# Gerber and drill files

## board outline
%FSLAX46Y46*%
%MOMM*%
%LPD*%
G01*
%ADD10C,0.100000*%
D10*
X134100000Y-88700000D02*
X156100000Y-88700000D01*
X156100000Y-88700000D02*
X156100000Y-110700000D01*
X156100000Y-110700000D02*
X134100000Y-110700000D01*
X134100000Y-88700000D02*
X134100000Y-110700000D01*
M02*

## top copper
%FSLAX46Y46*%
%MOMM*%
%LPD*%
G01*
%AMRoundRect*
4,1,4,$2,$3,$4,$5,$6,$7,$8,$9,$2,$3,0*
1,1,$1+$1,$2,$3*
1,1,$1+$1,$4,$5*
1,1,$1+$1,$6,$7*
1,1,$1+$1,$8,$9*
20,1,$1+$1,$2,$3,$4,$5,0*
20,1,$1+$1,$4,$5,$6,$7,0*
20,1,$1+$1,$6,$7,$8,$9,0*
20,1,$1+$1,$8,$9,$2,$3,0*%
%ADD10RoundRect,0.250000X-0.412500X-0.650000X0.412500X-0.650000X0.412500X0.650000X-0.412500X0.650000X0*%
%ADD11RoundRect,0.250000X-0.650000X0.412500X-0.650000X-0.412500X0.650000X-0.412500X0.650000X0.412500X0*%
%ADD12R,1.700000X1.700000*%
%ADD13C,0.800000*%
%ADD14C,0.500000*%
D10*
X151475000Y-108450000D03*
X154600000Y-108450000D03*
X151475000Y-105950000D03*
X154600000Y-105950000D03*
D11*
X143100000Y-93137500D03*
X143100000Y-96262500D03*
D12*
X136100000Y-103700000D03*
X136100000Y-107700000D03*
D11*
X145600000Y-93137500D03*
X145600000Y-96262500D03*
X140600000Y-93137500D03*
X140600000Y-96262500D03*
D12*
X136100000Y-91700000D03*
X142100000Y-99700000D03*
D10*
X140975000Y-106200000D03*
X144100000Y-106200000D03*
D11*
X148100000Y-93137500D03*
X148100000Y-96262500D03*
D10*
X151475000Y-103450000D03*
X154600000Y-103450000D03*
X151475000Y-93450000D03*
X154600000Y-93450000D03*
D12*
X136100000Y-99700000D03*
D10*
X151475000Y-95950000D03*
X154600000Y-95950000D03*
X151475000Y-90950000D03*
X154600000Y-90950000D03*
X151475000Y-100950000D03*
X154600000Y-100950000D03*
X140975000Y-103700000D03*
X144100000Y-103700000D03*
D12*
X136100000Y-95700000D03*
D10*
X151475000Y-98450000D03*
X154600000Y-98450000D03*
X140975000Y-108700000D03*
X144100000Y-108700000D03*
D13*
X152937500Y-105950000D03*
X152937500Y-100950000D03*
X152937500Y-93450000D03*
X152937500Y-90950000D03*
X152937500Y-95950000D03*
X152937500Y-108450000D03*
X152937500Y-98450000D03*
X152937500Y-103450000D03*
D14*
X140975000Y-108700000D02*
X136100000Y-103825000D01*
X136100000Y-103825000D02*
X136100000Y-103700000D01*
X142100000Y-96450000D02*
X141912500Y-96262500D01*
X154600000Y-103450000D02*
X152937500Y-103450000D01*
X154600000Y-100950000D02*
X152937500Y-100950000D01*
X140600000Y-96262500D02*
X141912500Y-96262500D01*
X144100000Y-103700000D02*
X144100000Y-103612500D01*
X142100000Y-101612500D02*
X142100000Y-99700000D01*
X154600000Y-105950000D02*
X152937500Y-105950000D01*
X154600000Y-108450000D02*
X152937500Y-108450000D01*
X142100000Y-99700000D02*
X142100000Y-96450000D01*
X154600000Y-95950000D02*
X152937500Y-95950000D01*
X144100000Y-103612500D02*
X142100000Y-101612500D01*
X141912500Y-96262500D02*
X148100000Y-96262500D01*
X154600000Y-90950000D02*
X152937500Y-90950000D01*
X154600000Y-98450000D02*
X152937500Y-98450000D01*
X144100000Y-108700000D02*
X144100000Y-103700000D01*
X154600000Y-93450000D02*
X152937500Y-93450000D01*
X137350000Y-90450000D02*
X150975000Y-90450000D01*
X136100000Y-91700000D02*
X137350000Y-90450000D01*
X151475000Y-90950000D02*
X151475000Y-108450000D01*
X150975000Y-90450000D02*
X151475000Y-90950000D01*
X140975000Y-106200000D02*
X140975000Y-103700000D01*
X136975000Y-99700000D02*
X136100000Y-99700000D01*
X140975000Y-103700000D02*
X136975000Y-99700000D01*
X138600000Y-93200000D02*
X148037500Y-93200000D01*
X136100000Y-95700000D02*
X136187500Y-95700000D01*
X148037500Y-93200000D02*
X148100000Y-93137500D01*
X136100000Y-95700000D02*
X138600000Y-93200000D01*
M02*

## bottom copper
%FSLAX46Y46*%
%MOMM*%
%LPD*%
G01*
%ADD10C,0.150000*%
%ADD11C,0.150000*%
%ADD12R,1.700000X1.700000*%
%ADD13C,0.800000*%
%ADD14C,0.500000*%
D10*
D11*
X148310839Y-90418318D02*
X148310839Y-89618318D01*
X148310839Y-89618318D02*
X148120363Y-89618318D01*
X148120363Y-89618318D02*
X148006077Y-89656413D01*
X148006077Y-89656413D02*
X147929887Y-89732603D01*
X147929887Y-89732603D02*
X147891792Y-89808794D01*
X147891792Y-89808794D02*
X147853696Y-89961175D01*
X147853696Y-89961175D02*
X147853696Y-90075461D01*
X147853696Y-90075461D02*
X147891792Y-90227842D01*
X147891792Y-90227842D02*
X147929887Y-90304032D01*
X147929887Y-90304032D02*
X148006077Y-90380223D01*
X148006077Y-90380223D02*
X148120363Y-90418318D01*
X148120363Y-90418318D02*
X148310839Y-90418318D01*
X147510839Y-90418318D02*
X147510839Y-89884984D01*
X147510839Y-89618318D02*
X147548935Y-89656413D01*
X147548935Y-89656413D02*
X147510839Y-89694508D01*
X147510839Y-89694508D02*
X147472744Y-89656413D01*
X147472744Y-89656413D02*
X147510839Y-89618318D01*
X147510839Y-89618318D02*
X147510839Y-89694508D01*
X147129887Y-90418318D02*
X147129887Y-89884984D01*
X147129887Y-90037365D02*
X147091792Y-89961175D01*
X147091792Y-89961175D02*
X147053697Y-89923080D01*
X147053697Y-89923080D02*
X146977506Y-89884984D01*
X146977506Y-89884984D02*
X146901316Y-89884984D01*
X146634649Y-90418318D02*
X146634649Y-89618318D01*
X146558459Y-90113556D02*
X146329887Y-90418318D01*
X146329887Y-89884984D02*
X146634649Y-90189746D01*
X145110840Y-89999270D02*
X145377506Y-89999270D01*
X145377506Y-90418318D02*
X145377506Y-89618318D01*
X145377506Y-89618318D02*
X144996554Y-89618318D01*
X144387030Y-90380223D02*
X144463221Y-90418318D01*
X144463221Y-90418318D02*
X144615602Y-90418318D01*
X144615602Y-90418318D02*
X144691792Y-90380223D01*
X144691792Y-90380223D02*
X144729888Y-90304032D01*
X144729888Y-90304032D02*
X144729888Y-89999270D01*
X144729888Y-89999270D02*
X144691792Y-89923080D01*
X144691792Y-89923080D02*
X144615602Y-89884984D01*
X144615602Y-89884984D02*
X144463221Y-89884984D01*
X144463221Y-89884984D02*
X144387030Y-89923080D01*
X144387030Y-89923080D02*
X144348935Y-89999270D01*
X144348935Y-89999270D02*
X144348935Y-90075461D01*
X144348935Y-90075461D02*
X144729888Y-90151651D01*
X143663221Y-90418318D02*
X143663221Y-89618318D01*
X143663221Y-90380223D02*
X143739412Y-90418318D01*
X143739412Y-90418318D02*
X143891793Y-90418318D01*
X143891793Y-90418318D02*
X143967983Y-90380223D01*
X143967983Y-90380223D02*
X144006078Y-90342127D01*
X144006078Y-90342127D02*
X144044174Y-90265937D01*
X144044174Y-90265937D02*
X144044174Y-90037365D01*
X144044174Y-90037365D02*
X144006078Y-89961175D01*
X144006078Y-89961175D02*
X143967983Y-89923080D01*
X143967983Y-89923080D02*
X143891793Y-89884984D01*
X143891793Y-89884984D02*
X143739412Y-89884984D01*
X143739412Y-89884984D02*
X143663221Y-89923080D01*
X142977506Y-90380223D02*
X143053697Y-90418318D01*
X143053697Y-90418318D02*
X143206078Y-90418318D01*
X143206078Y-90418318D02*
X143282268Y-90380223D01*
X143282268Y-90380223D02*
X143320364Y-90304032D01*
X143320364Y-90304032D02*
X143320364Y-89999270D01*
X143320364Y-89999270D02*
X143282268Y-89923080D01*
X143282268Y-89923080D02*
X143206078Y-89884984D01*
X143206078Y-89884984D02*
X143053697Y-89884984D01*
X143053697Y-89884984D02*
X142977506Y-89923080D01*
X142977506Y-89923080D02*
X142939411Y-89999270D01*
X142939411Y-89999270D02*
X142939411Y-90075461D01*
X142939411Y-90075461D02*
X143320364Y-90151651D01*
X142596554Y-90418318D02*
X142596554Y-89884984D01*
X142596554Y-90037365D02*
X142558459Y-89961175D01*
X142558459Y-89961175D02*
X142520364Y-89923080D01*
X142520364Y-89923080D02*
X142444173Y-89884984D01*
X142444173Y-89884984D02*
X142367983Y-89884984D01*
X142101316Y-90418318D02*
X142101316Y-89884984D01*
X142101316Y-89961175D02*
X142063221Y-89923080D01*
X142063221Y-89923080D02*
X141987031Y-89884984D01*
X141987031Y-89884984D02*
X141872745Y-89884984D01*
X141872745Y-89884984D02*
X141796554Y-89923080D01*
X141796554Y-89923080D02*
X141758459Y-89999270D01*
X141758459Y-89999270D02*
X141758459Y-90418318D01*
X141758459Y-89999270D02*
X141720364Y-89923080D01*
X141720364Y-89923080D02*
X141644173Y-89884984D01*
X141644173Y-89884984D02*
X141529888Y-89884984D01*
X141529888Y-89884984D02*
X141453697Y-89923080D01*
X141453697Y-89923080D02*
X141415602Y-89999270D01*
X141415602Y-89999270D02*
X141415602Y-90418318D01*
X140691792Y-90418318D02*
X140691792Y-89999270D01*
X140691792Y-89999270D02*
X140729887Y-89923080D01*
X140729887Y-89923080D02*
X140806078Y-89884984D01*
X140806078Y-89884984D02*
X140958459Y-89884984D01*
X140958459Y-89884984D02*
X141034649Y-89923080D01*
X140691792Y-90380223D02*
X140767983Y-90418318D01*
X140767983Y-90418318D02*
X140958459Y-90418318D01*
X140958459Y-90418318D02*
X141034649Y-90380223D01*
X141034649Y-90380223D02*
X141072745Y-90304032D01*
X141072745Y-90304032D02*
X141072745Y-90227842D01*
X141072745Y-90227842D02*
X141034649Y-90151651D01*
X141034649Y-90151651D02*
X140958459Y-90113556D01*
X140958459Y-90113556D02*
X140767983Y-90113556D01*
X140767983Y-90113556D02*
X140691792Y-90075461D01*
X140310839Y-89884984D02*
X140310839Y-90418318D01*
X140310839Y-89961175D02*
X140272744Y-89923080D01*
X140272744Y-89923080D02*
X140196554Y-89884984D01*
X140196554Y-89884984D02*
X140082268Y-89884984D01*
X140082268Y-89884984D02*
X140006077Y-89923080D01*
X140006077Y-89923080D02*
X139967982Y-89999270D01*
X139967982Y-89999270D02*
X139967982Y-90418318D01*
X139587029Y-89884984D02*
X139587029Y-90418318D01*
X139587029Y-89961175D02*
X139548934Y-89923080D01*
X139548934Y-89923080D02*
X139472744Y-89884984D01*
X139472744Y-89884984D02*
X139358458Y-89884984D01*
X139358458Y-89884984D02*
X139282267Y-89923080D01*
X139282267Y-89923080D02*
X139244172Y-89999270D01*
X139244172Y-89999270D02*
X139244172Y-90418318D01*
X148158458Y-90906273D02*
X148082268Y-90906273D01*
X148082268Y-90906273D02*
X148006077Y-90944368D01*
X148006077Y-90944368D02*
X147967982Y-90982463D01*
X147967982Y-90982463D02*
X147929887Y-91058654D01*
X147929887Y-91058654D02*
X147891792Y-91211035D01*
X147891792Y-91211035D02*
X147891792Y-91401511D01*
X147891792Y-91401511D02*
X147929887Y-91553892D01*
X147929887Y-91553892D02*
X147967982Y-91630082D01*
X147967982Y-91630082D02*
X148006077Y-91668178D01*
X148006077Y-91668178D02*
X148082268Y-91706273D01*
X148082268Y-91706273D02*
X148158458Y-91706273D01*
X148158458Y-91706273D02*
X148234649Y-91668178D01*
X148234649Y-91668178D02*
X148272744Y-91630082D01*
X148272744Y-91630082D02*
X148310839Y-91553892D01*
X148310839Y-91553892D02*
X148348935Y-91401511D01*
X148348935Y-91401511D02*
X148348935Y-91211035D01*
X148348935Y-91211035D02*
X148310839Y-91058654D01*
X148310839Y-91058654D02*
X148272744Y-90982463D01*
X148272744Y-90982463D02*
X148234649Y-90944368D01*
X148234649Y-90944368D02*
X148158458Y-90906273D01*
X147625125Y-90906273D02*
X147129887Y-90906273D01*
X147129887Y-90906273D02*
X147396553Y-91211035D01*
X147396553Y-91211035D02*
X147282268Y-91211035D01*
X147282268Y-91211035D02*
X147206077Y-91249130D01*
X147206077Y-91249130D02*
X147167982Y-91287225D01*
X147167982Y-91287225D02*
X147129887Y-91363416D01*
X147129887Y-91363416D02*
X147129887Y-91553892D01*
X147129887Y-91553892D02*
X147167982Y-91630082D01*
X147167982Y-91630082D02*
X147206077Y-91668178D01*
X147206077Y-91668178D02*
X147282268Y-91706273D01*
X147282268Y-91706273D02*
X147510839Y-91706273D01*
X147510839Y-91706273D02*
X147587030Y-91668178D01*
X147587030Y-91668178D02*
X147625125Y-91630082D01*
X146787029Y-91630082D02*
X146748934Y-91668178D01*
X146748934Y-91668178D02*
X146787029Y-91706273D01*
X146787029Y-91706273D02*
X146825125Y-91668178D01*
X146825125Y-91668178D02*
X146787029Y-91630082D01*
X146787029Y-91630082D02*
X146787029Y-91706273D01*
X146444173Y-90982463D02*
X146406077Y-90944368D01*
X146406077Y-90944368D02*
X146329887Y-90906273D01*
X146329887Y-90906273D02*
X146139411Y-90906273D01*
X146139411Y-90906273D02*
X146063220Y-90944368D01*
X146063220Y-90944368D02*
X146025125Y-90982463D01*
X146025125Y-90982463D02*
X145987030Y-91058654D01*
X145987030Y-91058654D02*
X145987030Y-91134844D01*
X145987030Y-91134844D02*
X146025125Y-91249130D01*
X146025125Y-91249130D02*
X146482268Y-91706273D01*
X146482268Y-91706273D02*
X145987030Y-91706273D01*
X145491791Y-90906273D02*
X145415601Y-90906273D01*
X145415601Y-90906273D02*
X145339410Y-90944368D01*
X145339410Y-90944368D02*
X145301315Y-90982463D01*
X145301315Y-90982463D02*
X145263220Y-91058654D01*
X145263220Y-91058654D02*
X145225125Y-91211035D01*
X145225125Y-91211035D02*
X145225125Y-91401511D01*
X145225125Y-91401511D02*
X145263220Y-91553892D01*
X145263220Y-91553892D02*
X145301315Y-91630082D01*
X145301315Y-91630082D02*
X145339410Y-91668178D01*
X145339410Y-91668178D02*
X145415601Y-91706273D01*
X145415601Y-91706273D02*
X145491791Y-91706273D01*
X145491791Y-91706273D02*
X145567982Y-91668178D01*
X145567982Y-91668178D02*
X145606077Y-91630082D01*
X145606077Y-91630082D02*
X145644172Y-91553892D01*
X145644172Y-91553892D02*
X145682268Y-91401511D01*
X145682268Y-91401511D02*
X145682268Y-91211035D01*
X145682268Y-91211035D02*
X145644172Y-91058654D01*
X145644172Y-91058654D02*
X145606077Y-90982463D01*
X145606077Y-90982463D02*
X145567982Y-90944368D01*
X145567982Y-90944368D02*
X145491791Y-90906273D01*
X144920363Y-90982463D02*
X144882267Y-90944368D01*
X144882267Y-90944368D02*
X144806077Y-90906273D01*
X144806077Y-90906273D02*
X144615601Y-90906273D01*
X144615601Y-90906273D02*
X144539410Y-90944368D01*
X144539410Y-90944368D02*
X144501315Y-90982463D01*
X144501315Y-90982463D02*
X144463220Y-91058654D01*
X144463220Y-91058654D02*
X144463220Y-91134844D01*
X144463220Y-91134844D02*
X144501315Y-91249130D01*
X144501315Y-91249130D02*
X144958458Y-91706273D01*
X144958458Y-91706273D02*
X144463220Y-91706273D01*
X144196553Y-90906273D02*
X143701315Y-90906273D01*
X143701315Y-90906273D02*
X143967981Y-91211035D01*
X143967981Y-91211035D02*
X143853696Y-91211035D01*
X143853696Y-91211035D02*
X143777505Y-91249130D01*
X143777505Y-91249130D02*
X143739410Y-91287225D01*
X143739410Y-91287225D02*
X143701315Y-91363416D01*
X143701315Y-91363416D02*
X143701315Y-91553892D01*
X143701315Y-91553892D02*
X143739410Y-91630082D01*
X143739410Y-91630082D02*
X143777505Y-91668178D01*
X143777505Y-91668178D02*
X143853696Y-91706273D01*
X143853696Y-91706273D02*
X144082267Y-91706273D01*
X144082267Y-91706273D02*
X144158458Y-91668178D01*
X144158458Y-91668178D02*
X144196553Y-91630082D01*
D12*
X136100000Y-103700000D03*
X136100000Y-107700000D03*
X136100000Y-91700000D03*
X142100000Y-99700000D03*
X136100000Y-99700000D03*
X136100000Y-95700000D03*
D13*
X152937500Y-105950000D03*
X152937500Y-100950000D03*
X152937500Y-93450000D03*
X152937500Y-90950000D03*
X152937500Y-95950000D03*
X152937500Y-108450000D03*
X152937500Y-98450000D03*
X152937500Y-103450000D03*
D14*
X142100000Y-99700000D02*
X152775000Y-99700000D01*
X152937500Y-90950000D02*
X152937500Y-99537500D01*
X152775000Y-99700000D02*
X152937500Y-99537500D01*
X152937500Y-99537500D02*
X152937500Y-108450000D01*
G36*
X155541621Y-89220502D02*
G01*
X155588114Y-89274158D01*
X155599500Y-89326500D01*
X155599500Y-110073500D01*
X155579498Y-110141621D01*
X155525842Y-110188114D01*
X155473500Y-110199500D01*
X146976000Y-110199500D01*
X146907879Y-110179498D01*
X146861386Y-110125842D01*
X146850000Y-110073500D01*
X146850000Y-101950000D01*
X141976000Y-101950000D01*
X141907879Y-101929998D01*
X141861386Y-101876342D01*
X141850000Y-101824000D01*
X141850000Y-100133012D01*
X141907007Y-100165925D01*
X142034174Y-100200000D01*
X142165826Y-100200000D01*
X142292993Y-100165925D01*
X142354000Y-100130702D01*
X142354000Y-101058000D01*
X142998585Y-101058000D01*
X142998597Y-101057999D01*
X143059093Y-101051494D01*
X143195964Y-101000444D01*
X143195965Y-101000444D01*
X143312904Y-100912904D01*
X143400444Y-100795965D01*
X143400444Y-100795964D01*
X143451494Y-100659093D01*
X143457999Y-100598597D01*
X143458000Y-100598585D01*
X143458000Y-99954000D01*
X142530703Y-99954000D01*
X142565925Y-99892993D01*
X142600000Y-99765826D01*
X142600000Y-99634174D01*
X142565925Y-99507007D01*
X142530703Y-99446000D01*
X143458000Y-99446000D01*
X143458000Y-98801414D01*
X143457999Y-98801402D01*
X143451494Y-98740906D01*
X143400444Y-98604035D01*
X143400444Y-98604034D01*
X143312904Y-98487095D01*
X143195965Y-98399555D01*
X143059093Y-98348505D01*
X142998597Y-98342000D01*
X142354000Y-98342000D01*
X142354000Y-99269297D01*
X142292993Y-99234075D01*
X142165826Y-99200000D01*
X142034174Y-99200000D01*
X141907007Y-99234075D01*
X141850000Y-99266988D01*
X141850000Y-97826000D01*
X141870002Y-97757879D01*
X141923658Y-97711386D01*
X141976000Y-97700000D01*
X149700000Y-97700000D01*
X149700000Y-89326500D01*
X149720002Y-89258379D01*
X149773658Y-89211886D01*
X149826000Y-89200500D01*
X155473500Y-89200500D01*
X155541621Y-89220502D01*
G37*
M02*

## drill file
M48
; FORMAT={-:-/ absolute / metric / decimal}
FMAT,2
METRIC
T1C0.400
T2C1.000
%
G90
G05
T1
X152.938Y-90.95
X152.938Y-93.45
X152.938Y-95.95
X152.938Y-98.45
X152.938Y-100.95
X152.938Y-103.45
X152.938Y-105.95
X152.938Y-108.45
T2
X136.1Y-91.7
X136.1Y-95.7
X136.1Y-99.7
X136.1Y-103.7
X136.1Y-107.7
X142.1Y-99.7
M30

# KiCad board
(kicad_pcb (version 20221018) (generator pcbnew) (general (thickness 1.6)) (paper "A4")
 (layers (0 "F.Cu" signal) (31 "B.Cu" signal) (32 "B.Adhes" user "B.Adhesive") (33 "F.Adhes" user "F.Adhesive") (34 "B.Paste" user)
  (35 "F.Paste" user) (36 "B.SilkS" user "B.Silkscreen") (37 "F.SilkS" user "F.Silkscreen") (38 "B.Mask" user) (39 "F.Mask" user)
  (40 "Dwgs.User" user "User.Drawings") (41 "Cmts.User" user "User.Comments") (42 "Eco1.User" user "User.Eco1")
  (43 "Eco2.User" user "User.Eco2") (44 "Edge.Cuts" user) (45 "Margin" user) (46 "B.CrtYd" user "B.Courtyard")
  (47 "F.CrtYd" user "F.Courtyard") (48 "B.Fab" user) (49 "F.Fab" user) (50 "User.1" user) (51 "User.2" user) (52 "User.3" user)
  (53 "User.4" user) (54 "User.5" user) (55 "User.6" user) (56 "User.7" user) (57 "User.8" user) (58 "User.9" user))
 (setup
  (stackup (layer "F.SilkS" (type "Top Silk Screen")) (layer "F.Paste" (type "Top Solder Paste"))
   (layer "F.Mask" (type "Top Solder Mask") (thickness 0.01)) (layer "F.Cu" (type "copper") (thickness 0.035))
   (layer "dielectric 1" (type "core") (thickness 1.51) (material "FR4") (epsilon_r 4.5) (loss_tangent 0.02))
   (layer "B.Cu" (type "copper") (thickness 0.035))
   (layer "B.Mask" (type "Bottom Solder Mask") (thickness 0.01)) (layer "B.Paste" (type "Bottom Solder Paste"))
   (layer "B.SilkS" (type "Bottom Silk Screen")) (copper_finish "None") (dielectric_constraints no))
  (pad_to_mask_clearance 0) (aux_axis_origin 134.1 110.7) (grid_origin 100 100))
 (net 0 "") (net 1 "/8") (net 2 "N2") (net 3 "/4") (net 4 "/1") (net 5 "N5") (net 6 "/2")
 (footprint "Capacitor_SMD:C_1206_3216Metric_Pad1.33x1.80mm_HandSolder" (layer "F.Cu") (at 153.0375 108.45)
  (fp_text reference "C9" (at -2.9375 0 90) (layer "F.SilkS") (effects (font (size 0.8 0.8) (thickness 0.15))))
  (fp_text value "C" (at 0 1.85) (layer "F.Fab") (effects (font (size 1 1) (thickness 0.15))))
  (pad "1" smd roundrect (at -1.5625 0) (size 1.325 1.8) (layers "F.Cu" "F.Paste" "F.Mask") (roundrect_rratio 0.1886792453) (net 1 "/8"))
  (pad "2" smd roundrect (at 1.5625 0) (size 1.325 1.8) (layers "F.Cu" "F.Paste" "F.Mask") (roundrect_rratio 0.1886792453) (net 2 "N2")))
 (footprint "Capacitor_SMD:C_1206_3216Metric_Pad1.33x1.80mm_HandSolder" (layer "F.Cu") (at 153.0375 105.95)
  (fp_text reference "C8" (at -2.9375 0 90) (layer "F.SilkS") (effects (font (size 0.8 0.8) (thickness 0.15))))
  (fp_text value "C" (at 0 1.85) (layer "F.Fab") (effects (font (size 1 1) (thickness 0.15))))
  (pad "1" smd roundrect (at -1.5625 0) (size 1.325 1.8) (layers "F.Cu" "F.Paste" "F.Mask") (roundrect_rratio 0.1886792453) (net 1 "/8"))
  (pad "2" smd roundrect (at 1.5625 0) (size 1.325 1.8) (layers "F.Cu" "F.Paste" "F.Mask") (roundrect_rratio 0.1886792453) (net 2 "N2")))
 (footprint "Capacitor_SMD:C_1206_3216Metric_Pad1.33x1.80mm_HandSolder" (layer "F.Cu") (at 143.1 94.7 -90)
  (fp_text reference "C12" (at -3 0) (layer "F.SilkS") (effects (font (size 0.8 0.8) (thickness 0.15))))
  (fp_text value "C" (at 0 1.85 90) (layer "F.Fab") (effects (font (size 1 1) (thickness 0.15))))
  (pad "1" smd roundrect (at -1.5625 0 270) (size 1.325 1.8) (layers "F.Cu" "F.Paste" "F.Mask") (roundrect_rratio 0.1886792453) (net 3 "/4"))
  (pad "2" smd roundrect (at 1.5625 0 270) (size 1.325 1.8) (layers "F.Cu" "F.Paste" "F.Mask") (roundrect_rratio 0.1886792453) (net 2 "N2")))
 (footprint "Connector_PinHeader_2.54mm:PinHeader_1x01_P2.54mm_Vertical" (layer "F.Cu") (at 136.1 103.7)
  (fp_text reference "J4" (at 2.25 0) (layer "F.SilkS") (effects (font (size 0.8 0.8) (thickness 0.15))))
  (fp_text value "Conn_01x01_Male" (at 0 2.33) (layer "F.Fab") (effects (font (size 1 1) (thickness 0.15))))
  (pad "1" thru_hole rect (at 0 0) (size 1.7 1.7) (drill 1) (layers "*.Cu" "*.Mask") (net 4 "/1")))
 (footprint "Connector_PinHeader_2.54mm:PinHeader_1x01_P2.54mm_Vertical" (layer "F.Cu") (at 136.1 107.7)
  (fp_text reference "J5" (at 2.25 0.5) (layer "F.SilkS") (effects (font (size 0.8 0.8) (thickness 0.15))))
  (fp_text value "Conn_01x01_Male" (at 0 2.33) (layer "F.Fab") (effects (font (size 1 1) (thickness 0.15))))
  (pad "1" thru_hole rect (at 0 0) (size 1.7 1.7) (drill 1) (layers "*.Cu" "*.Mask") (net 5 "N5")))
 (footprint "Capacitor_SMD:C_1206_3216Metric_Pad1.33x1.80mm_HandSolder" (layer "F.Cu") (at 145.6 94.7 -90)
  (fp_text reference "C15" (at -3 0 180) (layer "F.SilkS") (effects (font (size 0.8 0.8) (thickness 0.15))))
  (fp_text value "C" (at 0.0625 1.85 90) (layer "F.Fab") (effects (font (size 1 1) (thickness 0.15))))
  (pad "1" smd roundrect (at -1.5625 0 270) (size 1.325 1.8) (layers "F.Cu" "F.Paste" "F.Mask") (roundrect_rratio 0.1886792453) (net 3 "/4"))
  (pad "2" smd roundrect (at 1.5625 0 270) (size 1.325 1.8) (layers "F.Cu" "F.Paste" "F.Mask") (roundrect_rratio 0.1886792453) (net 2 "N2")))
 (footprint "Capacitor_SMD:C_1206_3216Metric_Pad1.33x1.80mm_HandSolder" (layer "F.Cu") (at 140.6 94.7 -90)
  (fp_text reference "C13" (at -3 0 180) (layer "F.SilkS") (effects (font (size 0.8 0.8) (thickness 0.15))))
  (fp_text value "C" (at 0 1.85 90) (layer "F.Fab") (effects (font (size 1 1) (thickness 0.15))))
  (pad "1" smd roundrect (at -1.5625 0 270) (size 1.325 1.8) (layers "F.Cu" "F.Paste" "F.Mask") (roundrect_rratio 0.1886792453) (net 3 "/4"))
  (pad "2" smd roundrect (at 1.5625 0 270) (size 1.325 1.8) (layers "F.Cu" "F.Paste" "F.Mask") (roundrect_rratio 0.1886792453) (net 2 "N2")))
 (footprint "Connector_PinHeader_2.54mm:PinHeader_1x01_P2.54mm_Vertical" (layer "F.Cu") (at 136.1 91.7)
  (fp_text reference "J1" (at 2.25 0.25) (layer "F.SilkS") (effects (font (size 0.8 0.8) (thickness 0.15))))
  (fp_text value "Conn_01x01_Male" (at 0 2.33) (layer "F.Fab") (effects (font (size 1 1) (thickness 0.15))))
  (pad "1" thru_hole rect (at 0 0) (size 1.7 1.7) (drill 1) (layers "*.Cu" "*.Mask") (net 1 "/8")))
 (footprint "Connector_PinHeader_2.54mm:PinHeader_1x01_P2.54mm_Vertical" (layer "F.Cu") (at 142.1 99.7)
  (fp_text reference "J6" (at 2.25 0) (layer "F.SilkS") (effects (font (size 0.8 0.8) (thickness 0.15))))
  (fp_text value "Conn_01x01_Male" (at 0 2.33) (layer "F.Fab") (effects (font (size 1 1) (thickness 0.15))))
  (pad "1" thru_hole rect (at 0 0) (size 1.7 1.7) (drill 1) (layers "*.Cu" "*.Mask") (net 2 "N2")))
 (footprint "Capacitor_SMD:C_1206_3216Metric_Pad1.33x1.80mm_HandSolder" (layer "F.Cu") (at 142.5375 106.2)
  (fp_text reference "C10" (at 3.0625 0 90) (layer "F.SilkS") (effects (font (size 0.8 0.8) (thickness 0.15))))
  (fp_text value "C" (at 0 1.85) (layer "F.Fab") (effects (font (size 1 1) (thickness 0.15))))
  (pad "1" smd roundrect (at -1.5625 0) (size 1.325 1.8) (layers "F.Cu" "F.Paste" "F.Mask") (roundrect_rratio 0.1886792453) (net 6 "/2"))
  (pad "2" smd roundrect (at 1.5625 0) (size 1.325 1.8) (layers "F.Cu" "F.Paste" "F.Mask") (roundrect_rratio 0.1886792453) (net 2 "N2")))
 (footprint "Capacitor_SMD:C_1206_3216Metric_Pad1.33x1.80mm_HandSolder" (layer "F.Cu") (at 148.1 94.7 -90)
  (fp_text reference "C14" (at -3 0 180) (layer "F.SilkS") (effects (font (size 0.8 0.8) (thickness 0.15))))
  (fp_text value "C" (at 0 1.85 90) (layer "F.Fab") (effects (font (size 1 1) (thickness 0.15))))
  (pad "1" smd roundrect (at -1.5625 0 270) (size 1.325 1.8) (layers "F.Cu" "F.Paste" "F.Mask") (roundrect_rratio 0.1886792453) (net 3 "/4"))
  (pad "2" smd roundrect (at 1.5625 0 270) (size 1.325 1.8) (layers "F.Cu" "F.Paste" "F.Mask") (roundrect_rratio 0.1886792453) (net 2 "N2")))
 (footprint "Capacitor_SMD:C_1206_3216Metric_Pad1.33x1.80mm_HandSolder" (layer "F.Cu") (at 153.0375 103.45)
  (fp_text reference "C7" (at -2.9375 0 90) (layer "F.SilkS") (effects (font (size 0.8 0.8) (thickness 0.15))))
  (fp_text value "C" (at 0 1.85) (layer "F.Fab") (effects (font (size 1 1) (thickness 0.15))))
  (pad "1" smd roundrect (at -1.5625 0) (size 1.325 1.8) (layers "F.Cu" "F.Paste" "F.Mask") (roundrect_rratio 0.1886792453) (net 1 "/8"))
  (pad "2" smd roundrect (at 1.5625 0) (size 1.325 1.8) (layers "F.Cu" "F.Paste" "F.Mask") (roundrect_rratio 0.1886792453) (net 2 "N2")))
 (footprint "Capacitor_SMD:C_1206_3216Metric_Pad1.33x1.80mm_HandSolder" (layer "F.Cu") (at 153.0375 93.45)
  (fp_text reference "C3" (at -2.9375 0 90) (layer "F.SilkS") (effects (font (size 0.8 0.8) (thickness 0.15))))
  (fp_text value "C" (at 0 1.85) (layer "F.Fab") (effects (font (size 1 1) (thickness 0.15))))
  (pad "1" smd roundrect (at -1.5625 0) (size 1.325 1.8) (layers "F.Cu" "F.Paste" "F.Mask") (roundrect_rratio 0.1886792453) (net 1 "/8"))
  (pad "2" smd roundrect (at 1.5625 0) (size 1.325 1.8) (layers "F.Cu" "F.Paste" "F.Mask") (roundrect_rratio 0.1886792453) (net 2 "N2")))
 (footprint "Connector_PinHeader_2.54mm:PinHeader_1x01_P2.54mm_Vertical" (layer "F.Cu") (at 136.1 99.7)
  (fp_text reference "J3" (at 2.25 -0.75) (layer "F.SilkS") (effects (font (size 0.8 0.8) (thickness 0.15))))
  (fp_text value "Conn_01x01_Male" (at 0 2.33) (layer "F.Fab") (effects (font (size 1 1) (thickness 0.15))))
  (pad "1" thru_hole rect (at 0 0) (size 1.7 1.7) (drill 1) (layers "*.Cu" "*.Mask") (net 6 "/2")))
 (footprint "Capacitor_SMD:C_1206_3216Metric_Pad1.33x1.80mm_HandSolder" (layer "F.Cu") (at 153.0375 95.95)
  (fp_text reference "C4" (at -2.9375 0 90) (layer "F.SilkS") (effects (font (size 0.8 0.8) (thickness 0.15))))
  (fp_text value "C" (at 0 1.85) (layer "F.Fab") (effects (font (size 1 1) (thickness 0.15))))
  (pad "1" smd roundrect (at -1.5625 0) (size 1.325 1.8) (layers "F.Cu" "F.Paste" "F.Mask") (roundrect_rratio 0.1886792453) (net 1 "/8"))
  (pad "2" smd roundrect (at 1.5625 0) (size 1.325 1.8) (layers "F.Cu" "F.Paste" "F.Mask") (roundrect_rratio 0.1886792453) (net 2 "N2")))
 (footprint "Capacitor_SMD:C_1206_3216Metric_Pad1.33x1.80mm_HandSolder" (layer "F.Cu") (at 153.0375 90.95)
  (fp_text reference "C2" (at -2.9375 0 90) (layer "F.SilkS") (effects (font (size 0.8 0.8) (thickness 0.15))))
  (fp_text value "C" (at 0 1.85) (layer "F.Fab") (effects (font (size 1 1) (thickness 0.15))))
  (pad "1" smd roundrect (at -1.5625 0) (size 1.325 1.8) (layers "F.Cu" "F.Paste" "F.Mask") (roundrect_rratio 0.1886792453) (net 1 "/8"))
  (pad "2" smd roundrect (at 1.5625 0) (size 1.325 1.8) (layers "F.Cu" "F.Paste" "F.Mask") (roundrect_rratio 0.1886792453) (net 2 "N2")))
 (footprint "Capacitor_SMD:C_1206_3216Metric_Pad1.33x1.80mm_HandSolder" (layer "F.Cu") (at 153.0375 100.95)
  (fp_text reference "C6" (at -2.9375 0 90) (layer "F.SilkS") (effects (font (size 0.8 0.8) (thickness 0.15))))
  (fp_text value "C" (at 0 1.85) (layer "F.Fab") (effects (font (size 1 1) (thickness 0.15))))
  (pad "1" smd roundrect (at -1.5625 0) (size 1.325 1.8) (layers "F.Cu" "F.Paste" "F.Mask") (roundrect_rratio 0.1886792453) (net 1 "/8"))
  (pad "2" smd roundrect (at 1.5625 0) (size 1.325 1.8) (layers "F.Cu" "F.Paste" "F.Mask") (roundrect_rratio 0.1886792453) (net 2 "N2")))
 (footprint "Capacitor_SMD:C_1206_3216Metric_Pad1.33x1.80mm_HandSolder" (layer "F.Cu") (at 142.5375 103.7)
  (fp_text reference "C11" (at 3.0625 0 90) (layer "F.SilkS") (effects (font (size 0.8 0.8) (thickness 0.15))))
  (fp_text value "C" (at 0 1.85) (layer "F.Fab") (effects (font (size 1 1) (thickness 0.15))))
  (pad "1" smd roundrect (at -1.5625 0) (size 1.325 1.8) (layers "F.Cu" "F.Paste" "F.Mask") (roundrect_rratio 0.1886792453) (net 6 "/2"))
  (pad "2" smd roundrect (at 1.5625 0) (size 1.325 1.8) (layers "F.Cu" "F.Paste" "F.Mask") (roundrect_rratio 0.1886792453) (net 2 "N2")))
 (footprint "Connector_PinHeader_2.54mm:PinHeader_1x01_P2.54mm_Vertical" (layer "F.Cu") (at 136.1 95.7)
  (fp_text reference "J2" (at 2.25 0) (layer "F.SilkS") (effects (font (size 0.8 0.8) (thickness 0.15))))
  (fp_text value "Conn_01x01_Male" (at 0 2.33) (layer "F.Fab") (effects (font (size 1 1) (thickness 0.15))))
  (pad "1" thru_hole rect (at 0 0) (size 1.7 1.7) (drill 1) (layers "*.Cu" "*.Mask") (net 3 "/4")))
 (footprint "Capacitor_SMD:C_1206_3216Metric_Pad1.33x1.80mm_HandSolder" (layer "F.Cu") (at 153.0375 98.45)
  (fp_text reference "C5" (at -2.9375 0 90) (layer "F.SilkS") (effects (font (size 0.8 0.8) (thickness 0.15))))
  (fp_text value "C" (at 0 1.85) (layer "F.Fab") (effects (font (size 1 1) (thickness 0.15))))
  (pad "1" smd roundrect (at -1.5625 0) (size 1.325 1.8) (layers "F.Cu" "F.Paste" "F.Mask") (roundrect_rratio 0.1886792453) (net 1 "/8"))
  (pad "2" smd roundrect (at 1.5625 0) (size 1.325 1.8) (layers "F.Cu" "F.Paste" "F.Mask") (roundrect_rratio 0.1886792453) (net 2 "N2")))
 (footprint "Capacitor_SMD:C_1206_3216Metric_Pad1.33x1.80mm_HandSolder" (layer "F.Cu") (at 142.5375 108.7)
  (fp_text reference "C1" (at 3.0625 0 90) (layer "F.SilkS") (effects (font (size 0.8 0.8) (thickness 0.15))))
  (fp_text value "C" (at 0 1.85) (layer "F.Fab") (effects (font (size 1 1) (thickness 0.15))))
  (pad "1" smd roundrect (at -1.5625 0) (size 1.325 1.8) (layers "F.Cu" "F.Paste" "F.Mask") (roundrect_rratio 0.1886792453) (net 4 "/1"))
  (pad "2" smd roundrect (at 1.5625 0) (size 1.325 1.8) (layers "F.Cu" "F.Paste" "F.Mask") (roundrect_rratio 0.1886792453) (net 2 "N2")))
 (gr_line (start 134.1 88.7) (end 156.1 88.7) (stroke (width 0.1) (type solid)) (layer "Edge.Cuts"))
 (gr_line (start 156.1 88.7) (end 156.1 110.7) (stroke (width 0.1) (type solid)) (layer "Edge.Cuts"))
 (gr_line (start 156.1 110.7) (end 134.1 110.7) (stroke (width 0.1) (type solid)) (layer "Edge.Cuts"))
 (gr_line (start 134.1 88.7) (end 134.1 110.7) (stroke (width 0.1) (type solid)) (layer "Edge.Cuts"))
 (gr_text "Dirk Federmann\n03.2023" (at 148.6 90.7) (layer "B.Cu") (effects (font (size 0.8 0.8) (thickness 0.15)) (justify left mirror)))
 (segment (start 140.975 108.7) (end 136.1 103.825) (width 0.5) (layer "F.Cu") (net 4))
 (segment (start 136.1 103.825) (end 136.1 103.7) (width 0.5) (layer "F.Cu") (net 4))
 (segment (start 142.1 96.45) (end 141.9125 96.2625) (width 0.5) (layer "F.Cu") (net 2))
 (segment (start 154.6 103.45) (end 152.9375 103.45) (width 0.5) (layer "F.Cu") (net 2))
 (segment (start 154.6 100.95) (end 152.9375 100.95) (width 0.5) (layer "F.Cu") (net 2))
 (segment (start 140.6 96.2625) (end 141.9125 96.2625) (width 0.5) (layer "F.Cu") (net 2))
 (segment (start 144.1 103.7) (end 144.1 103.6125) (width 0.5) (layer "F.Cu") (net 2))
 (segment (start 142.1 101.6125) (end 142.1 99.7) (width 0.5) (layer "F.Cu") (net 2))
 (segment (start 154.6 105.95) (end 152.9375 105.95) (width 0.5) (layer "F.Cu") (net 2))
 (segment (start 154.6 108.45) (end 152.9375 108.45) (width 0.5) (layer "F.Cu") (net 2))
 (segment (start 142.1 99.7) (end 142.1 96.45) (width 0.5) (layer "F.Cu") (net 2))
 (segment (start 154.6 95.95) (end 152.9375 95.95) (width 0.5) (layer "F.Cu") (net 2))
 (segment (start 144.1 103.6125) (end 142.1 101.6125) (width 0.5) (layer "F.Cu") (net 2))
 (segment (start 141.9125 96.2625) (end 148.1 96.2625) (width 0.5) (layer "F.Cu") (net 2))
 (segment (start 154.6 90.95) (end 152.9375 90.95) (width 0.5) (layer "F.Cu") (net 2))
 (segment (start 154.6 98.45) (end 152.9375 98.45) (width 0.5) (layer "F.Cu") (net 2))
 (segment (start 144.1 108.7) (end 144.1 103.7) (width 0.5) (layer "F.Cu") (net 2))
 (segment (start 154.6 93.45) (end 152.9375 93.45) (width 0.5) (layer "F.Cu") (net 2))
 (via (at 152.9375 105.95) (size 0.8) (drill 0.4) (layers "F.Cu" "B.Cu") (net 2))
 (via (at 152.9375 100.95) (size 0.8) (drill 0.4) (layers "F.Cu" "B.Cu") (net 2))
 (via (at 152.9375 93.45) (size 0.8) (drill 0.4) (layers "F.Cu" "B.Cu") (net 2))
 (via (at 152.9375 90.95) (size 0.8) (drill 0.4) (layers "F.Cu" "B.Cu") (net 2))
 (via (at 152.9375 95.95) (size 0.8) (drill 0.4) (layers "F.Cu" "B.Cu") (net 2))
 (via (at 152.9375 108.45) (size 0.8) (drill 0.4) (layers "F.Cu" "B.Cu") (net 2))
 (via (at 152.9375 98.45) (size 0.8) (drill 0.4) (layers "F.Cu" "B.Cu") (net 2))
 (via (at 152.9375 103.45) (size 0.8) (drill 0.4) (layers "F.Cu" "B.Cu") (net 2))
 (segment (start 142.1 99.7) (end 152.775 99.7) (width 0.5) (layer "B.Cu") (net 2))
 (segment (start 152.9375 90.95) (end 152.9375 99.5375) (width 0.5) (layer "B.Cu") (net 2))
 (segment (start 152.775 99.7) (end 152.9375 99.5375) (width 0.5) (layer "B.Cu") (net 2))
 (segment (start 152.9375 99.5375) (end 152.9375 108.45) (width 0.5) (layer "B.Cu") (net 2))
 (segment (start 137.35 90.45) (end 150.975 90.45) (width 0.5) (layer "F.Cu") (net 1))
 (segment (start 136.1 91.7) (end 137.35 90.45) (width 0.5) (layer "F.Cu") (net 1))
 (segment (start 151.475 90.95) (end 151.475 108.45) (width 0.5) (layer "F.Cu") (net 1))
 (segment (start 150.975 90.45) (end 151.475 90.95) (width 0.5) (layer "F.Cu") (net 1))
 (segment (start 140.975 106.2) (end 140.975 103.7) (width 0.5) (layer "F.Cu") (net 6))
 (segment (start 136.975 99.7) (end 136.1 99.7) (width 0.5) (layer "F.Cu") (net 6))
 (segment (start 140.975 103.7) (end 136.975 99.7) (width 0.5) (layer "F.Cu") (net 6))
 (segment (start 138.6 93.2) (end 148.0375 93.2) (width 0.5) (layer "F.Cu") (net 3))
 (segment (start 136.1 95.7) (end 136.1875 95.7) (width 0.5) (layer "F.Cu") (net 3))
 (segment (start 148.0375 93.2) (end 148.1 93.1375) (width 0.5) (layer "F.Cu") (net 3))
 (segment (start 136.1 95.7) (end 138.6 93.2) (width 0.5) (layer "F.Cu") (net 3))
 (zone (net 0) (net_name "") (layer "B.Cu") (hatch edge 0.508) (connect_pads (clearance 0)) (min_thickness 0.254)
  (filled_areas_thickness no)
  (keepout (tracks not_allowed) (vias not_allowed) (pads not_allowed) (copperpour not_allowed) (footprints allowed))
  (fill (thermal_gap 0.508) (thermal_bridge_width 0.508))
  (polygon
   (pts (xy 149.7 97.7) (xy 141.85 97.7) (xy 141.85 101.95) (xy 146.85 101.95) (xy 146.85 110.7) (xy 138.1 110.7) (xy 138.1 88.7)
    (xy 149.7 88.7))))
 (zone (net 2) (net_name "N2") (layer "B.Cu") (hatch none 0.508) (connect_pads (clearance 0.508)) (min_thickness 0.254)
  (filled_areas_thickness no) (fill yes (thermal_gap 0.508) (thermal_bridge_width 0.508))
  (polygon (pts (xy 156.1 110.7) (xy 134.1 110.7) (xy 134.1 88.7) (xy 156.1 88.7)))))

